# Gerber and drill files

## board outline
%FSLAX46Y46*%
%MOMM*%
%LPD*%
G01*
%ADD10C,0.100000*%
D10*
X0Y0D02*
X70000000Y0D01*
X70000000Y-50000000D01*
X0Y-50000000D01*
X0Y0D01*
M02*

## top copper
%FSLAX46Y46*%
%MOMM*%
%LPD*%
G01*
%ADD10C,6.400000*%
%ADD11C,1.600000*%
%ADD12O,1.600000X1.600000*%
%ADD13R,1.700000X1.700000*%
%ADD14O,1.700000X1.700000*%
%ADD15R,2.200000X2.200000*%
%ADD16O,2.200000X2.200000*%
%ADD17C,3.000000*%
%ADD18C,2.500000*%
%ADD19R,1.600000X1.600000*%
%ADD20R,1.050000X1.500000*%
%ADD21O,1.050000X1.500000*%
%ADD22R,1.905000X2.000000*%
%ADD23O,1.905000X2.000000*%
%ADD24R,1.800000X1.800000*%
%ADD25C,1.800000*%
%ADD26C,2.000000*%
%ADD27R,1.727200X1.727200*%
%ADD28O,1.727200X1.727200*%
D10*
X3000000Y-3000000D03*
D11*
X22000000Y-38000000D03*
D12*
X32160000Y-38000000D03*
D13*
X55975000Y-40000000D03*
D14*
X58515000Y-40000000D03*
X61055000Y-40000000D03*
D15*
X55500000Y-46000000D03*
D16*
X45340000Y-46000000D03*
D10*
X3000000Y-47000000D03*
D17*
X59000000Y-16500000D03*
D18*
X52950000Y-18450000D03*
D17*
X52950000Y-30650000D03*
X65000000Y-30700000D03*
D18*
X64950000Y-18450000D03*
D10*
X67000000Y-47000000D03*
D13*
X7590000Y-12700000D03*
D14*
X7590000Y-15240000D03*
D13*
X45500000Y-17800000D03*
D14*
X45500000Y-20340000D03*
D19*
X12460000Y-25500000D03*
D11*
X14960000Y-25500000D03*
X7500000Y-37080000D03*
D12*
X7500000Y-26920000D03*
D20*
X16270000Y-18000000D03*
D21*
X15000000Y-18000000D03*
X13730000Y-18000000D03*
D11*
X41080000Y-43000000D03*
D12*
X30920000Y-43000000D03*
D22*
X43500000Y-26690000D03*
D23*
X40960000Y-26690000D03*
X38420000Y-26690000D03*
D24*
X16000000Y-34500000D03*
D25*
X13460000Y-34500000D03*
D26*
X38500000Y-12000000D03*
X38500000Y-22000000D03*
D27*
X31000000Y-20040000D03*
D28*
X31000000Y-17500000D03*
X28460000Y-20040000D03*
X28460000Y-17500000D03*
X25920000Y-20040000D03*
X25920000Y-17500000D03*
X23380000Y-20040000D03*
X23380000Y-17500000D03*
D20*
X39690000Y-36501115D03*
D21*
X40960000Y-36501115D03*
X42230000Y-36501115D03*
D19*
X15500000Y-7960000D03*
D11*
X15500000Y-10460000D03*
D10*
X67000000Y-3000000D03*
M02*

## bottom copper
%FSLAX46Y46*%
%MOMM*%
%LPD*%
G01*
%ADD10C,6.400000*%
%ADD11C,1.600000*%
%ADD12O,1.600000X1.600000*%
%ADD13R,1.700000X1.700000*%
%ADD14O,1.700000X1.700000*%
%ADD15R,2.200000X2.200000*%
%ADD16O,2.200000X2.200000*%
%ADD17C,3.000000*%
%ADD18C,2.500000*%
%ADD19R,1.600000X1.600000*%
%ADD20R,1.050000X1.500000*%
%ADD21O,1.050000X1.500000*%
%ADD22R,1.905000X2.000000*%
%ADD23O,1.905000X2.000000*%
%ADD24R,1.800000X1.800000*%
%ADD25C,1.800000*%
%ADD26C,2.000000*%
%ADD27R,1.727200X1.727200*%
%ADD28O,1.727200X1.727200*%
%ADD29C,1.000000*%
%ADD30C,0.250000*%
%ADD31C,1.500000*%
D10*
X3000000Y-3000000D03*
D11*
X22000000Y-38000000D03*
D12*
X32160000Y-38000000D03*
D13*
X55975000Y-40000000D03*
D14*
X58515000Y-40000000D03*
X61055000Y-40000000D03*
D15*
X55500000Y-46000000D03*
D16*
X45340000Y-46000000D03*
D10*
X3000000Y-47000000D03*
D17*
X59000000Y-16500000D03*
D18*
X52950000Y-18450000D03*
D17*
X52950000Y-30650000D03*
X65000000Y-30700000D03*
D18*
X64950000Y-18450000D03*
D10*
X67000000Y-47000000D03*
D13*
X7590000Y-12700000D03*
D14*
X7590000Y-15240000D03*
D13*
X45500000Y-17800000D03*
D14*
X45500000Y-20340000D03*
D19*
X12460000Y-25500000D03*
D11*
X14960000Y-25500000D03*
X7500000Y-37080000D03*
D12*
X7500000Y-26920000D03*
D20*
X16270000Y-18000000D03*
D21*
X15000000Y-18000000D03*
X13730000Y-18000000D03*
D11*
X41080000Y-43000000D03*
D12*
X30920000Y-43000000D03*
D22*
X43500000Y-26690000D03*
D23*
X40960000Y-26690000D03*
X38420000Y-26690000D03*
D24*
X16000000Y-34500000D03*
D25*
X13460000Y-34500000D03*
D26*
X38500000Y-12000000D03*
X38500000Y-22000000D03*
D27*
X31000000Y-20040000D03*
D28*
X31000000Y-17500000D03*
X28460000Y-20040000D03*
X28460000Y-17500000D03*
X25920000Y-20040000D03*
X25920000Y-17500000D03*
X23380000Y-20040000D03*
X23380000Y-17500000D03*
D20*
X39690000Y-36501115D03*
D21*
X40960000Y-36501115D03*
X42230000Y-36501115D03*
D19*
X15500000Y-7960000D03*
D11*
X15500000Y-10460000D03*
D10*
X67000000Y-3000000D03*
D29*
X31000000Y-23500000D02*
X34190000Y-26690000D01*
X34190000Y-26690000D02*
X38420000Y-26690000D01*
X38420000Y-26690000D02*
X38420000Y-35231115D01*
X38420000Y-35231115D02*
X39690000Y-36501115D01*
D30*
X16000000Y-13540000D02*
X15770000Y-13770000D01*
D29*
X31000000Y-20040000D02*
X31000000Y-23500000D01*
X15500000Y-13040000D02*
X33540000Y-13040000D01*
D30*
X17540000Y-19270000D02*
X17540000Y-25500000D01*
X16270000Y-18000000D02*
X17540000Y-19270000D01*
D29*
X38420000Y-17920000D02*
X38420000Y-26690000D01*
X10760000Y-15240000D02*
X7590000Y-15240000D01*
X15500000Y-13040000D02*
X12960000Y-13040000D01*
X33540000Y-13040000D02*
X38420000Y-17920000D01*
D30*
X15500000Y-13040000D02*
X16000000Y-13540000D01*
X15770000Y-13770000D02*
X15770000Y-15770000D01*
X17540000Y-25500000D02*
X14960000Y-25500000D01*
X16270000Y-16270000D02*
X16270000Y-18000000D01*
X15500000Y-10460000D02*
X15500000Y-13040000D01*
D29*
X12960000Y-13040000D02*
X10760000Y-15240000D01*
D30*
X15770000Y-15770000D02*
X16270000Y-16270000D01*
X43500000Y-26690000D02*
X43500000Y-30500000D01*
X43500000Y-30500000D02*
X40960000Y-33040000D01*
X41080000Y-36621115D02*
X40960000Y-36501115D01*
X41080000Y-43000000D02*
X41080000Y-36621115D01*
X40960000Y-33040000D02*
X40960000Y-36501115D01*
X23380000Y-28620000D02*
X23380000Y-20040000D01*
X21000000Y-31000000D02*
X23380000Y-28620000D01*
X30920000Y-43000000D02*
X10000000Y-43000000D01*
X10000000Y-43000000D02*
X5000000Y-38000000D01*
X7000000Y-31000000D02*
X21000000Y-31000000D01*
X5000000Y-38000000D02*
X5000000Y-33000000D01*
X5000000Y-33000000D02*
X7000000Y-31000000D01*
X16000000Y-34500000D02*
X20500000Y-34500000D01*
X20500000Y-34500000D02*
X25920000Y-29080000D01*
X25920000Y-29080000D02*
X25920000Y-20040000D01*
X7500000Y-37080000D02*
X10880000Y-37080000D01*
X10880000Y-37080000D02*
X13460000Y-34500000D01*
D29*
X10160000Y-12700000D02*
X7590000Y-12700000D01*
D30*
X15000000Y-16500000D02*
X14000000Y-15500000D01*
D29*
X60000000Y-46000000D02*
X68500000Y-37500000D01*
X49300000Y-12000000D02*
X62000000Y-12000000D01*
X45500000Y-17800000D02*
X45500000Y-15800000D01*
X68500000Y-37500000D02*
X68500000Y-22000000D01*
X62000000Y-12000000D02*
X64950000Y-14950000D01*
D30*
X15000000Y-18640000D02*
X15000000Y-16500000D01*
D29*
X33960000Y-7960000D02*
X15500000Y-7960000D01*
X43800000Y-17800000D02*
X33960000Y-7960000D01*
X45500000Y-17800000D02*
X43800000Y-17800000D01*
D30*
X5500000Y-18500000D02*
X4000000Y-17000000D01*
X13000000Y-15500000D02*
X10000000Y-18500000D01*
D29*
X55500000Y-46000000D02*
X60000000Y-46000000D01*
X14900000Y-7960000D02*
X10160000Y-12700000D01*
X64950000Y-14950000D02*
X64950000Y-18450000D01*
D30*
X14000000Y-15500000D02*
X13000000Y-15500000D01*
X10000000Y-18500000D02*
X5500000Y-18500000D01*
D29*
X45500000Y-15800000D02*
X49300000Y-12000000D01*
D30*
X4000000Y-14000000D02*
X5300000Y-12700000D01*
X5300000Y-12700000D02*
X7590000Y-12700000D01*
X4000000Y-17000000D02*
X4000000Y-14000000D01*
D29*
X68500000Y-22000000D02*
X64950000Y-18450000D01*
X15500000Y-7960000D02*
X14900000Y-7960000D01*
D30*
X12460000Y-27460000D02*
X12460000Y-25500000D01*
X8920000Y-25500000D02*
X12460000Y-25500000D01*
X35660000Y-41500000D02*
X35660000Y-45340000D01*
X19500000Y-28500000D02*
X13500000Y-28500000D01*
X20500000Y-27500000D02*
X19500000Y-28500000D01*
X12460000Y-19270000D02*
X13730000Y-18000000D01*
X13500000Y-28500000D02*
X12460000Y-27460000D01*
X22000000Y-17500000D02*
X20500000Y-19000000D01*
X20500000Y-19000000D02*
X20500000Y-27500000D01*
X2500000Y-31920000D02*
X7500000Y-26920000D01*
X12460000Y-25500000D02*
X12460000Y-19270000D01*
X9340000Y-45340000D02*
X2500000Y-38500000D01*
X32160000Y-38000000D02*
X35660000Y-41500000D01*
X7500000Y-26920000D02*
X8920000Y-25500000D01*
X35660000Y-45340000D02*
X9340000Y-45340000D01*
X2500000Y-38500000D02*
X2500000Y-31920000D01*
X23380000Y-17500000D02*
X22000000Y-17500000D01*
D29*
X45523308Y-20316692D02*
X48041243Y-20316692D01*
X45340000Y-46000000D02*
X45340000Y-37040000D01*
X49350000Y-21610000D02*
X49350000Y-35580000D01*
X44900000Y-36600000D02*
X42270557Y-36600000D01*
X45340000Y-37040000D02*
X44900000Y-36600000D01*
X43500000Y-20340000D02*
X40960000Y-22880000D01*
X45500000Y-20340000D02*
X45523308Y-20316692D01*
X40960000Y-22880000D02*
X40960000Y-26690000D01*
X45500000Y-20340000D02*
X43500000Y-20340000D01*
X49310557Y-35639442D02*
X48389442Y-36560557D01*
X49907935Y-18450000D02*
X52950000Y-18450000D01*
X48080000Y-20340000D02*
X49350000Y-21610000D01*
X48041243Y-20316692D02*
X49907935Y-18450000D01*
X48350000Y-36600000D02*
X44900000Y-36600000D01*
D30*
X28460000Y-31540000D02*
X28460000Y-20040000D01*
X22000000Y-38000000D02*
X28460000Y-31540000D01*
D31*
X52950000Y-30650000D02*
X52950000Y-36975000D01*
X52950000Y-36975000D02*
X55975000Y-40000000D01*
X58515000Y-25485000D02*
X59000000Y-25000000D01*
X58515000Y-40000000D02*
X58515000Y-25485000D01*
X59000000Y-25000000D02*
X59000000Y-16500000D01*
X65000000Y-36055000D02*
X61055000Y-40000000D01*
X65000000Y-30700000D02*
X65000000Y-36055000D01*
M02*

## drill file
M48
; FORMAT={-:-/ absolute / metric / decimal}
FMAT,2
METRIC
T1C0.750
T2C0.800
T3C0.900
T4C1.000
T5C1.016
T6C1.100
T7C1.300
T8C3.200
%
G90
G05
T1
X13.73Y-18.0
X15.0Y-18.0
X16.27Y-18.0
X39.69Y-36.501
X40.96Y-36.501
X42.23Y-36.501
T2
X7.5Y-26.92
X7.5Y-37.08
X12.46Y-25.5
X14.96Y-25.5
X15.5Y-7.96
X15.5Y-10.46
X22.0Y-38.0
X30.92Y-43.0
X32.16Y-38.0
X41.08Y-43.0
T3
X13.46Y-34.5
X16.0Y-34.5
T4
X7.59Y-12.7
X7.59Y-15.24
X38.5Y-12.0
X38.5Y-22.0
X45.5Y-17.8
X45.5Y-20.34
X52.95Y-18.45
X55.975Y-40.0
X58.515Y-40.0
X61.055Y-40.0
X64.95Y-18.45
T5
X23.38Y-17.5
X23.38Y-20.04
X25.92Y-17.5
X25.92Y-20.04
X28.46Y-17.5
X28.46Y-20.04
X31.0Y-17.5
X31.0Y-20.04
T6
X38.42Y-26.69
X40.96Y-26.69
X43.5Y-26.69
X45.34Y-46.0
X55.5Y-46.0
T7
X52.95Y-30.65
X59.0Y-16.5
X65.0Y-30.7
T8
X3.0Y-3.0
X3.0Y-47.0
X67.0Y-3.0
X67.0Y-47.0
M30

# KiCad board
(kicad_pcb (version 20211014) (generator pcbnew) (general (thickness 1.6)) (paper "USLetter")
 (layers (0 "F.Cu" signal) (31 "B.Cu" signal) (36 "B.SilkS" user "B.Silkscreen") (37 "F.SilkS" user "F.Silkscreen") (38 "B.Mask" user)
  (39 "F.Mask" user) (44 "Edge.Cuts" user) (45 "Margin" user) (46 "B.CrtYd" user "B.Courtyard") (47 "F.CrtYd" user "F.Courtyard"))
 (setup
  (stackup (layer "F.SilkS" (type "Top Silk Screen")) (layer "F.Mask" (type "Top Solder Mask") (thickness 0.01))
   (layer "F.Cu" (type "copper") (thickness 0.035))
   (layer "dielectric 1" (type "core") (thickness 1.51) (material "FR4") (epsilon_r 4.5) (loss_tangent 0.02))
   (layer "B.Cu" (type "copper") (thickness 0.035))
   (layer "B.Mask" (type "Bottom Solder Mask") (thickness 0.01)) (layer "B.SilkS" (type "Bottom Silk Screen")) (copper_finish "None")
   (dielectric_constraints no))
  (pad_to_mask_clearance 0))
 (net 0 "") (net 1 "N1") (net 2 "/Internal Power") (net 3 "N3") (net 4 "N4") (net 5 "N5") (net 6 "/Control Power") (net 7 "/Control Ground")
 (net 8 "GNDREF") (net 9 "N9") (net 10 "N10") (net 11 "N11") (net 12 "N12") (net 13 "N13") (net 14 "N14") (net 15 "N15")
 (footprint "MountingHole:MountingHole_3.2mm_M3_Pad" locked (layer "F.Cu") (at 3 3)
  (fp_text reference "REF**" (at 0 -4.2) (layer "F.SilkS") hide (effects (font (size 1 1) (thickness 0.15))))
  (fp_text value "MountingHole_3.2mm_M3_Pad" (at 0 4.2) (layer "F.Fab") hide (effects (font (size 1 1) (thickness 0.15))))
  (pad "1" thru_hole circle locked (at 0 0) (size 6.4 6.4) (drill 3.2) (layers *.Cu *.Mask)))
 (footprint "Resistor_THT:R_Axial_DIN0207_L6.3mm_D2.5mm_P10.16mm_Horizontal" (layer "F.Cu") (at 22 38)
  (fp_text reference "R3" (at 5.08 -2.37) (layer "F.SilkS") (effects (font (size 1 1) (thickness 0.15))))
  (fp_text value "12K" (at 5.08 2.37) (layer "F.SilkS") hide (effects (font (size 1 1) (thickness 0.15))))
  (pad "1" thru_hole circle (at 0 0) (size 1.6 1.6) (drill 0.8) (layers *.Cu *.Mask) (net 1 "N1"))
  (pad "2" thru_hole oval (at 10.16 0) (size 1.6 1.6) (drill 0.8) (layers *.Cu *.Mask) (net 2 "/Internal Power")))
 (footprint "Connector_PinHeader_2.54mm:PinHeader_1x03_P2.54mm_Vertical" (layer "F.Cu") (at 55.975 40 90)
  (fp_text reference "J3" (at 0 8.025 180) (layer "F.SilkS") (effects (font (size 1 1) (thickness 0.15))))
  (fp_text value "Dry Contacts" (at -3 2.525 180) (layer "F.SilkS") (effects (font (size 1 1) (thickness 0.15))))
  (pad "1" thru_hole rect (at 0 0 90) (size 1.7 1.7) (drill 1) (layers *.Cu *.Mask) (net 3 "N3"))
  (pad "2" thru_hole oval (at 0 2.54 90) (size 1.7 1.7) (drill 1) (layers *.Cu *.Mask) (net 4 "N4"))
  (pad "3" thru_hole oval (at 0 5.08 90) (size 1.7 1.7) (drill 1) (layers *.Cu *.Mask) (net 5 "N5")))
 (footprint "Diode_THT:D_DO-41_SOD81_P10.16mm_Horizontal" (layer "F.Cu") (at 55.5 46 180)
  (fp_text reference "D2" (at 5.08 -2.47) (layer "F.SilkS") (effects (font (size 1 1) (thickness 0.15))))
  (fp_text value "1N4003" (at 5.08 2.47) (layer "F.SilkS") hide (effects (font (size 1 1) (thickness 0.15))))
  (pad "1" thru_hole rect (at 0 0 180) (size 2.2 2.2) (drill 1.1) (layers *.Cu *.Mask) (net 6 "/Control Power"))
  (pad "2" thru_hole oval (at 10.16 0 180) (size 2.2 2.2) (drill 1.1) (layers *.Cu *.Mask) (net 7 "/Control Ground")))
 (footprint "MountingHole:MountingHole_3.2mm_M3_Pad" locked (layer "F.Cu") (at 3 47)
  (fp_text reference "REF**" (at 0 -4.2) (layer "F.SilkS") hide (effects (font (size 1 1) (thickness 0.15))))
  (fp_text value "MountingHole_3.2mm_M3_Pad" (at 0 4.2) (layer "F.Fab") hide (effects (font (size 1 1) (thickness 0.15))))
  (pad "1" thru_hole circle locked (at 0 0) (size 6.4 6.4) (drill 3.2) (layers *.Cu *.Mask)))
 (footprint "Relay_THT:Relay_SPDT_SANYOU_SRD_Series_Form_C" (layer "F.Cu") (at 59 16.5 -90)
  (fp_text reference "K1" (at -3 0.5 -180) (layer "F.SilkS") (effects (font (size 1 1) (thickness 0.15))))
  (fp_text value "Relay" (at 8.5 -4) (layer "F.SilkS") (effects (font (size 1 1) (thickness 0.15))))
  (pad "1" thru_hole circle (at 0 0) (size 3 3) (drill 1.3) (layers *.Cu *.Mask) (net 4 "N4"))
  (pad "2" thru_hole circle (at 1.95 6.05) (size 2.5 2.5) (drill 1) (layers *.Cu *.Mask) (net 7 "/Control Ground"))
  (pad "3" thru_hole circle (at 14.15 6.05) (size 3 3) (drill 1.3) (layers *.Cu *.Mask) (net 3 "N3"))
  (pad "4" thru_hole circle (at 14.2 -6) (size 3 3) (drill 1.3) (layers *.Cu *.Mask) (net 5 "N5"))
  (pad "5" thru_hole circle (at 1.95 -5.95) (size 2.5 2.5) (drill 1) (layers *.Cu *.Mask) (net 6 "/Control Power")))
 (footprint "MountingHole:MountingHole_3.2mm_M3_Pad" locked (layer "F.Cu") (at 67 47)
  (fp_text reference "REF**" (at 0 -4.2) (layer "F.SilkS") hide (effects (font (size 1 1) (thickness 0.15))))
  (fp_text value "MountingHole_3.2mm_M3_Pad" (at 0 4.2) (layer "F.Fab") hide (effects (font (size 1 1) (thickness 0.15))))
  (pad "1" thru_hole circle locked (at 0 0) (size 6.4 6.4) (drill 3.2) (layers *.Cu *.Mask)))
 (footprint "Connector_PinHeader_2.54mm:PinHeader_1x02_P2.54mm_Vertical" (layer "F.Cu") (at 7.59 12.7)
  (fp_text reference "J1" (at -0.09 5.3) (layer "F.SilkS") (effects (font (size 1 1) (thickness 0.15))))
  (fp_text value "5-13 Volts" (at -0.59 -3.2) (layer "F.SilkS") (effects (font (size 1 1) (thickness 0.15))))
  (pad "1" thru_hole rect (at 0 0) (size 1.7 1.7) (drill 1) (layers *.Cu *.Mask) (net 6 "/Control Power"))
  (pad "2" thru_hole oval (at 0 2.54) (size 1.7 1.7) (drill 1) (layers *.Cu *.Mask) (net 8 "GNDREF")))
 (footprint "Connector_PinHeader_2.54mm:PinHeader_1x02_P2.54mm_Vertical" (layer "F.Cu") (at 45.5 17.8)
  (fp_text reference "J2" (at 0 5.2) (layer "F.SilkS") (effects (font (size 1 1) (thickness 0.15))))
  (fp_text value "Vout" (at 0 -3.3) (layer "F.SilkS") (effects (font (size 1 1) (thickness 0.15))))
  (pad "1" thru_hole rect (at 0 0) (size 1.7 1.7) (drill 1) (layers *.Cu *.Mask) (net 6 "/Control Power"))
  (pad "2" thru_hole oval (at 0 2.54) (size 1.7 1.7) (drill 1) (layers *.Cu *.Mask) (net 7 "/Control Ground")))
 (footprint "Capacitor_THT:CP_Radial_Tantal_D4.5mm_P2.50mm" (layer "F.Cu") (at 12.46 25.5)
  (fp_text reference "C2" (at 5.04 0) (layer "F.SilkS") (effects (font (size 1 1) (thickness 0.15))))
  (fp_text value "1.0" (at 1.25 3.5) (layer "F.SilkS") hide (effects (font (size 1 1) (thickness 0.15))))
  (pad "1" thru_hole rect (at 0 0) (size 1.6 1.6) (drill 0.8) (layers *.Cu *.Mask) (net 2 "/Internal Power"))
  (pad "2" thru_hole circle (at 2.5 0) (size 1.6 1.6) (drill 0.8) (layers *.Cu *.Mask) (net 8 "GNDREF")))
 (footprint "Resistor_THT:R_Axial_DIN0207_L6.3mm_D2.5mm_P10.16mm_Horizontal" (layer "F.Cu") (at 7.5 37.08 90)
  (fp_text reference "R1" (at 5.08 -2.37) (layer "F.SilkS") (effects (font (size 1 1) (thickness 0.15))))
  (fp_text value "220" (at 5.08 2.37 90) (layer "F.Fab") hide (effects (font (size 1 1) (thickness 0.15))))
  (pad "1" thru_hole circle (at 0 0 90) (size 1.6 1.6) (drill 0.8) (layers *.Cu *.Mask) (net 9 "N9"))
  (pad "2" thru_hole oval (at 10.16 0 90) (size 1.6 1.6) (drill 0.8) (layers *.Cu *.Mask) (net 2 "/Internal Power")))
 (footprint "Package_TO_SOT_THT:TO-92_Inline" (layer "F.Cu") (at 16.27 18 180)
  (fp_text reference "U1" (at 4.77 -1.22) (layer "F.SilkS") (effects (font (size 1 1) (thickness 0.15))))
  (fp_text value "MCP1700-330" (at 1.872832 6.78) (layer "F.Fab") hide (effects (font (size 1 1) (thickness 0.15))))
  (pad "1" thru_hole rect (at 0 0 180) (size 1.05 1.5) (drill 0.75) (layers *.Cu *.Mask) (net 8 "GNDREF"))
  (pad "2" thru_hole oval (at 1.27 0 180) (size 1.05 1.5) (drill 0.75) (layers *.Cu *.Mask) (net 6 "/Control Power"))
  (pad "3" thru_hole oval (at 2.54 0 180) (size 1.05 1.5) (drill 0.75) (layers *.Cu *.Mask) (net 2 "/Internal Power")))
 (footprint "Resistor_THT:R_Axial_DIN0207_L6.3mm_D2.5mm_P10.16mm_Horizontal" (layer "F.Cu") (at 41.08 43 180)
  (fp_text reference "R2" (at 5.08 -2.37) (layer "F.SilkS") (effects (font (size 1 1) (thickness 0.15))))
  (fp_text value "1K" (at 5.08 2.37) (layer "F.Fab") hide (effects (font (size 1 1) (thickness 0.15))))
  (pad "1" thru_hole circle (at 0 0 180) (size 1.6 1.6) (drill 0.8) (layers *.Cu *.Mask) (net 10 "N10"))
  (pad "2" thru_hole oval (at 10.16 0 180) (size 1.6 1.6) (drill 0.8) (layers *.Cu *.Mask) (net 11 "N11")))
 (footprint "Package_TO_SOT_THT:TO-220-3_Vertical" (layer "F.Cu") (at 43.5 26.69 180)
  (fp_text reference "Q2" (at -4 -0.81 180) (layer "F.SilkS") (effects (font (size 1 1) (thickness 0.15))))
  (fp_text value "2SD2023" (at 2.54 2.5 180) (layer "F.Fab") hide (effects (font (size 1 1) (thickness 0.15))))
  (pad "1" thru_hole rect (at 0 0 180) (size 1.905 2) (drill 1.1) (layers *.Cu *.Mask) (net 10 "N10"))
  (pad "2" thru_hole oval (at 2.54 0 180) (size 1.905 2) (drill 1.1) (layers *.Cu *.Mask) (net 7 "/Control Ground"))
  (pad "3" thru_hole oval (at 5.08 0 180) (size 1.905 2) (drill 1.1) (layers *.Cu *.Mask) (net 8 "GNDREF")))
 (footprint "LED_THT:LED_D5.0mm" (layer "F.Cu") (at 16 34.5 180)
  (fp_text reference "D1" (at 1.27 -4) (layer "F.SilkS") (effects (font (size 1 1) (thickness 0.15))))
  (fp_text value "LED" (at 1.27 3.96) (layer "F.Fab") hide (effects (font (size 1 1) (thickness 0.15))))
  (pad "1" thru_hole rect (at 0 0 180) (size 1.8 1.8) (drill 0.9) (layers *.Cu *.Mask) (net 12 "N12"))
  (pad "2" thru_hole circle (at 2.54 0 180) (size 1.8 1.8) (drill 0.9) (layers *.Cu *.Mask) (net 9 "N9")))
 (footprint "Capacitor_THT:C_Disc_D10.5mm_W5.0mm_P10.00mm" (layer "F.Cu") (at 38.5 12 -90)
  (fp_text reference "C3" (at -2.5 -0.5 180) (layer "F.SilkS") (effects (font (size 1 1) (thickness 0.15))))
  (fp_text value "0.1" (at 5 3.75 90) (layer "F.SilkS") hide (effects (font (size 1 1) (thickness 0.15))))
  (pad "1" thru_hole circle (at 0 0 270) (size 2 2) (drill 1) (layers *.Cu *.Mask) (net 6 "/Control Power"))
  (pad "2" thru_hole circle (at 10 0 270) (size 2 2) (drill 1) (layers *.Cu *.Mask) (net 8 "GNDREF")))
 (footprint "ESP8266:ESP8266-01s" (layer "F.Cu") (at 31 17.5 -90)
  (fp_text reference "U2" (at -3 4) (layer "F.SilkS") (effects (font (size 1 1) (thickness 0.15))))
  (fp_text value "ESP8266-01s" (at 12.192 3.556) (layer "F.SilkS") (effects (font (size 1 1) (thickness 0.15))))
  (pad "1" thru_hole rect (at 2.54 0 270) (size 1.7272 1.7272) (drill 1.016) (layers *.Cu *.Mask) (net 8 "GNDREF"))
  (pad "2" thru_hole oval (at 0 0 270) (size 1.7272 1.7272) (drill 1.016) (layers *.Cu *.Mask) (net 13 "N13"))
  (pad "3" thru_hole oval (at 2.54 2.54 270) (size 1.7272 1.7272) (drill 1.016) (layers *.Cu *.Mask) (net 1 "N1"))
  (pad "4" thru_hole oval (at 0 2.54 270) (size 1.7272 1.7272) (drill 1.016) (layers *.Cu *.Mask) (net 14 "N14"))
  (pad "5" thru_hole oval (at 2.54 5.08 270) (size 1.7272 1.7272) (drill 1.016) (layers *.Cu *.Mask) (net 12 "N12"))
  (pad "6" thru_hole oval (at 0 5.08 270) (size 1.7272 1.7272) (drill 1.016) (layers *.Cu *.Mask) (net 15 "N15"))
  (pad "7" thru_hole oval (at 2.54 7.62 270) (size 1.7272 1.7272) (drill 1.016) (layers *.Cu *.Mask) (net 11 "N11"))
  (pad "8" thru_hole oval (at 0 7.62 270) (size 1.7272 1.7272) (drill 1.016) (layers *.Cu *.Mask) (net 2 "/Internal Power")))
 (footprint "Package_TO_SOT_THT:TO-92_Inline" (layer "F.Cu") (at 39.69 36.501115)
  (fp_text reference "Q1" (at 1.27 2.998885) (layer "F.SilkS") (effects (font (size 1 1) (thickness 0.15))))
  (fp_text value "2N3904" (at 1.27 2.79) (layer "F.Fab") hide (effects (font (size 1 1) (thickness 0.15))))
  (pad "1" thru_hole rect (at 0 0) (size 1.05 1.5) (drill 0.75) (layers *.Cu *.Mask) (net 8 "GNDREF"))
  (pad "2" thru_hole oval (at 1.27 0) (size 1.05 1.5) (drill 0.75) (layers *.Cu *.Mask) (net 10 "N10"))
  (pad "3" thru_hole oval (at 2.54 0) (size 1.05 1.5) (drill 0.75) (layers *.Cu *.Mask) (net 7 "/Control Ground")))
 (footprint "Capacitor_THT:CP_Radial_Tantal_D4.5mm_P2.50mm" (layer "F.Cu") (at 15.5 7.96 -90)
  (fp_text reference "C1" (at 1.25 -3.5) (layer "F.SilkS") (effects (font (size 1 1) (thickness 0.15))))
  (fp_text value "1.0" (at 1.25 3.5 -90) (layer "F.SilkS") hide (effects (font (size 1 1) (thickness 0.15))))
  (pad "1" thru_hole rect (at 0 0 270) (size 1.6 1.6) (drill 0.8) (layers *.Cu *.Mask) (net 6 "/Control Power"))
  (pad "2" thru_hole circle (at 2.5 0 270) (size 1.6 1.6) (drill 0.8) (layers *.Cu *.Mask) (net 8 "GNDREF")))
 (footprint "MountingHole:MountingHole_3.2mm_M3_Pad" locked (layer "F.Cu") (at 67 3)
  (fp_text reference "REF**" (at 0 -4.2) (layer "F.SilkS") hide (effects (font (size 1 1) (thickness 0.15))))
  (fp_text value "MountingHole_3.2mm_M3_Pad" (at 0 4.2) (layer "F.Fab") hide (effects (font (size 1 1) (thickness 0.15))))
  (pad "1" thru_hole circle locked (at 0 0) (size 6.4 6.4) (drill 3.2) (layers *.Cu *.Mask)))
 (gr_rect locked (start 0 0) (end 70 50) (layer "Edge.Cuts") (width 0.1) (fill none))
 (segment (start 31 23.5) (end 34.19 26.69) (width 1) (layer "B.Cu") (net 8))
 (segment (start 34.19 26.69) (end 38.42 26.69) (width 1) (layer "B.Cu") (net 8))
 (segment (start 38.42 26.69) (end 38.42 35.231115) (width 1) (layer "B.Cu") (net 8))
 (segment (start 38.42 35.231115) (end 39.69 36.501115) (width 1) (layer "B.Cu") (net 8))
 (segment (start 16 13.54) (end 15.77 13.77) (width 0.25) (layer "B.Cu") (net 8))
 (segment (start 31 20.04) (end 31 23.5) (width 1) (layer "B.Cu") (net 8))
 (segment (start 15.5 13.04) (end 33.54 13.04) (width 1) (layer "B.Cu") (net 8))
 (segment (start 17.54 19.27) (end 17.54 25.5) (width 0.25) (layer "B.Cu") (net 8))
 (segment (start 16.27 18) (end 17.54 19.27) (width 0.25) (layer "B.Cu") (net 8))
 (segment (start 38.42 17.92) (end 38.42 26.69) (width 1) (layer "B.Cu") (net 8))
 (segment (start 10.76 15.24) (end 7.59 15.24) (width 1) (layer "B.Cu") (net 8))
 (segment (start 15.5 13.04) (end 12.96 13.04) (width 1) (layer "B.Cu") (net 8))
 (segment (start 33.54 13.04) (end 38.42 17.92) (width 1) (layer "B.Cu") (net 8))
 (segment (start 15.5 13.04) (end 16 13.54) (width 0.25) (layer "B.Cu") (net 8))
 (segment (start 15.77 13.77) (end 15.77 15.77) (width 0.25) (layer "B.Cu") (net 8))
 (segment (start 17.54 25.5) (end 14.96 25.5) (width 0.25) (layer "B.Cu") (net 8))
 (segment (start 16.27 16.27) (end 16.27 18) (width 0.25) (layer "B.Cu") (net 8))
 (segment (start 15.5 10.46) (end 15.5 13.04) (width 0.25) (layer "B.Cu") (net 8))
 (segment (start 12.96 13.04) (end 10.76 15.24) (width 1) (layer "B.Cu") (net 8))
 (segment (start 15.77 15.77) (end 16.27 16.27) (width 0.25) (layer "B.Cu") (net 8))
 (segment (start 43.5 26.69) (end 43.5 30.5) (width 0.25) (layer "B.Cu") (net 10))
 (segment (start 43.5 30.5) (end 40.96 33.04) (width 0.25) (layer "B.Cu") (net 10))
 (segment (start 41.08 36.621115) (end 40.96 36.501115) (width 0.25) (layer "B.Cu") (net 10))
 (segment (start 41.08 43) (end 41.08 36.621115) (width 0.25) (layer "B.Cu") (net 10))
 (segment (start 40.96 33.04) (end 40.96 36.501115) (width 0.25) (layer "B.Cu") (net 10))
 (segment (start 23.38 28.62) (end 23.38 20.04) (width 0.25) (layer "B.Cu") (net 11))
 (segment (start 21 31) (end 23.38 28.62) (width 0.25) (layer "B.Cu") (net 11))
 (segment (start 30.92 43) (end 10 43) (width 0.25) (layer "B.Cu") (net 11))
 (segment (start 10 43) (end 5 38) (width 0.25) (layer "B.Cu") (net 11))
 (segment (start 7 31) (end 21 31) (width 0.25) (layer "B.Cu") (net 11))
 (segment (start 5 38) (end 5 33) (width 0.25) (layer "B.Cu") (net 11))
 (segment (start 5 33) (end 7 31) (width 0.25) (layer "B.Cu") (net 11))
 (segment (start 16 34.5) (end 20.5 34.5) (width 0.25) (layer "B.Cu") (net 12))
 (segment (start 20.5 34.5) (end 25.92 29.08) (width 0.25) (layer "B.Cu") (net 12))
 (segment (start 25.92 29.08) (end 25.92 20.04) (width 0.25) (layer "B.Cu") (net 12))
 (segment (start 7.5 37.08) (end 10.88 37.08) (width 0.25) (layer "B.Cu") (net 9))
 (segment (start 10.88 37.08) (end 13.46 34.5) (width 0.25) (layer "B.Cu") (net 9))
 (segment (start 10.16 12.7) (end 7.59 12.7) (width 1) (layer "B.Cu") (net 6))
 (segment (start 15 16.5) (end 14 15.5) (width 0.25) (layer "B.Cu") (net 6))
 (segment (start 60 46) (end 68.5 37.5) (width 1) (layer "B.Cu") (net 6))
 (segment (start 49.3 12) (end 62 12) (width 1) (layer "B.Cu") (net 6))
 (segment (start 45.5 17.8) (end 45.5 15.8) (width 1) (layer "B.Cu") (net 6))
 (segment (start 68.5 37.5) (end 68.5 22) (width 1) (layer "B.Cu") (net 6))
 (segment (start 62 12) (end 64.95 14.95) (width 1) (layer "B.Cu") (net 6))
 (segment (start 15 18.64) (end 15 16.5) (width 0.25) (layer "B.Cu") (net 6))
 (segment (start 33.96 7.96) (end 15.5 7.96) (width 1) (layer "B.Cu") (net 6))
 (segment (start 43.8 17.8) (end 33.96 7.96) (width 1) (layer "B.Cu") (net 6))
 (segment (start 45.5 17.8) (end 43.8 17.8) (width 1) (layer "B.Cu") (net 6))
 (segment (start 5.5 18.5) (end 4 17) (width 0.25) (layer "B.Cu") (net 6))
 (segment (start 13 15.5) (end 10 18.5) (width 0.25) (layer "B.Cu") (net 6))
 (segment (start 55.5 46) (end 60 46) (width 1) (layer "B.Cu") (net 6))
 (segment (start 14.9 7.96) (end 10.16 12.7) (width 1) (layer "B.Cu") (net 6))
 (segment (start 64.95 14.95) (end 64.95 18.45) (width 1) (layer "B.Cu") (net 6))
 (segment (start 14 15.5) (end 13 15.5) (width 0.25) (layer "B.Cu") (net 6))
 (segment (start 10 18.5) (end 5.5 18.5) (width 0.25) (layer "B.Cu") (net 6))
 (segment (start 45.5 15.8) (end 49.3 12) (width 1) (layer "B.Cu") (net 6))
 (segment (start 4 14) (end 5.3 12.7) (width 0.25) (layer "B.Cu") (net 6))
 (segment (start 5.3 12.7) (end 7.59 12.7) (width 0.25) (layer "B.Cu") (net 6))
 (segment (start 4 17) (end 4 14) (width 0.25) (layer "B.Cu") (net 6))
 (segment (start 68.5 22) (end 64.95 18.45) (width 1) (layer "B.Cu") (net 6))
 (segment (start 15.5 7.96) (end 14.9 7.96) (width 1) (layer "B.Cu") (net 6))
 (segment (start 12.46 27.46) (end 12.46 25.5) (width 0.25) (layer "B.Cu") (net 2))
 (segment (start 8.92 25.5) (end 12.46 25.5) (width 0.25) (layer "B.Cu") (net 2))
 (segment (start 35.66 41.5) (end 35.66 45.34) (width 0.25) (layer "B.Cu") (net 2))
 (segment (start 19.5 28.5) (end 13.5 28.5) (width 0.25) (layer "B.Cu") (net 2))
 (segment (start 20.5 27.5) (end 19.5 28.5) (width 0.25) (layer "B.Cu") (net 2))
 (segment (start 12.46 19.27) (end 13.73 18) (width 0.25) (layer "B.Cu") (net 2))
 (segment (start 13.5 28.5) (end 12.46 27.46) (width 0.25) (layer "B.Cu") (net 2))
 (segment (start 22 17.5) (end 20.5 19) (width 0.25) (layer "B.Cu") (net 2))
 (segment (start 20.5 19) (end 20.5 27.5) (width 0.25) (layer "B.Cu") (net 2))
 (segment (start 2.5 31.92) (end 7.5 26.92) (width 0.25) (layer "B.Cu") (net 2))
 (segment (start 12.46 25.5) (end 12.46 19.27) (width 0.25) (layer "B.Cu") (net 2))
 (segment (start 9.34 45.34) (end 2.5 38.5) (width 0.25) (layer "B.Cu") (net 2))
 (segment (start 32.16 38) (end 35.66 41.5) (width 0.25) (layer "B.Cu") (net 2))
 (segment (start 7.5 26.92) (end 8.92 25.5) (width 0.25) (layer "B.Cu") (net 2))
 (segment (start 35.66 45.34) (end 9.34 45.34) (width 0.25) (layer "B.Cu") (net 2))
 (segment (start 2.5 38.5) (end 2.5 31.92) (width 0.25) (layer "B.Cu") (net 2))
 (segment (start 23.38 17.5) (end 22 17.5) (width 0.25) (layer "B.Cu") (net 2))
 (segment (start 45.523308 20.316692) (end 48.041243 20.316692) (width 1) (layer "B.Cu") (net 7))
 (segment (start 45.34 46) (end 45.34 37.04) (width 1) (layer "B.Cu") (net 7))
 (segment (start 49.35 21.61) (end 49.35 35.58) (width 1) (layer "B.Cu") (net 7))
 (segment (start 44.9 36.6) (end 42.270557 36.6) (width 1) (layer "B.Cu") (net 7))
 (segment (start 45.34 37.04) (end 44.9 36.6) (width 1) (layer "B.Cu") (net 7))
 (segment (start 43.5 20.34) (end 40.96 22.88) (width 1) (layer "B.Cu") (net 7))
 (segment (start 45.5 20.34) (end 45.523308 20.316692) (width 1) (layer "B.Cu") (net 7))
 (segment (start 40.96 22.88) (end 40.96 26.69) (width 1) (layer "B.Cu") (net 7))
 (segment (start 45.5 20.34) (end 43.5 20.34) (width 1) (layer "B.Cu") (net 7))
 (segment (start 49.310557 35.639442) (end 48.389442 36.560557) (width 1) (layer "B.Cu") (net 7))
 (segment (start 49.907935 18.45) (end 52.95 18.45) (width 1) (layer "B.Cu") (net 7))
 (segment (start 48.08 20.34) (end 49.35 21.61) (width 1) (layer "B.Cu") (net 7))
 (segment (start 48.041243 20.316692) (end 49.907935 18.45) (width 1) (layer "B.Cu") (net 7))
 (segment (start 48.35 36.6) (end 44.9 36.6) (width 1) (layer "B.Cu") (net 7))
 (segment (start 28.46 31.54) (end 28.46 20.04) (width 0.25) (layer "B.Cu") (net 1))
 (segment (start 22 38) (end 28.46 31.54) (width 0.25) (layer "B.Cu") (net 1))
 (segment (start 52.95 30.65) (end 52.95 36.975) (width 1.5) (layer "B.Cu") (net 3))
 (segment (start 52.95 36.975) (end 55.975 40) (width 1.5) (layer "B.Cu") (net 3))
 (segment (start 58.515 25.485) (end 59 25) (width 1.5) (layer "B.Cu") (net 4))
 (segment (start 58.515 40) (end 58.515 25.485) (width 1.5) (layer "B.Cu") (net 4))
 (segment (start 59 25) (end 59 16.5) (width 1.5) (layer "B.Cu") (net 4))
 (segment (start 65 36.055) (end 61.055 40) (width 1.5) (layer "B.Cu") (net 5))
 (segment (start 65 30.7) (end 65 36.055) (width 1.5) (layer "B.Cu") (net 5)))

